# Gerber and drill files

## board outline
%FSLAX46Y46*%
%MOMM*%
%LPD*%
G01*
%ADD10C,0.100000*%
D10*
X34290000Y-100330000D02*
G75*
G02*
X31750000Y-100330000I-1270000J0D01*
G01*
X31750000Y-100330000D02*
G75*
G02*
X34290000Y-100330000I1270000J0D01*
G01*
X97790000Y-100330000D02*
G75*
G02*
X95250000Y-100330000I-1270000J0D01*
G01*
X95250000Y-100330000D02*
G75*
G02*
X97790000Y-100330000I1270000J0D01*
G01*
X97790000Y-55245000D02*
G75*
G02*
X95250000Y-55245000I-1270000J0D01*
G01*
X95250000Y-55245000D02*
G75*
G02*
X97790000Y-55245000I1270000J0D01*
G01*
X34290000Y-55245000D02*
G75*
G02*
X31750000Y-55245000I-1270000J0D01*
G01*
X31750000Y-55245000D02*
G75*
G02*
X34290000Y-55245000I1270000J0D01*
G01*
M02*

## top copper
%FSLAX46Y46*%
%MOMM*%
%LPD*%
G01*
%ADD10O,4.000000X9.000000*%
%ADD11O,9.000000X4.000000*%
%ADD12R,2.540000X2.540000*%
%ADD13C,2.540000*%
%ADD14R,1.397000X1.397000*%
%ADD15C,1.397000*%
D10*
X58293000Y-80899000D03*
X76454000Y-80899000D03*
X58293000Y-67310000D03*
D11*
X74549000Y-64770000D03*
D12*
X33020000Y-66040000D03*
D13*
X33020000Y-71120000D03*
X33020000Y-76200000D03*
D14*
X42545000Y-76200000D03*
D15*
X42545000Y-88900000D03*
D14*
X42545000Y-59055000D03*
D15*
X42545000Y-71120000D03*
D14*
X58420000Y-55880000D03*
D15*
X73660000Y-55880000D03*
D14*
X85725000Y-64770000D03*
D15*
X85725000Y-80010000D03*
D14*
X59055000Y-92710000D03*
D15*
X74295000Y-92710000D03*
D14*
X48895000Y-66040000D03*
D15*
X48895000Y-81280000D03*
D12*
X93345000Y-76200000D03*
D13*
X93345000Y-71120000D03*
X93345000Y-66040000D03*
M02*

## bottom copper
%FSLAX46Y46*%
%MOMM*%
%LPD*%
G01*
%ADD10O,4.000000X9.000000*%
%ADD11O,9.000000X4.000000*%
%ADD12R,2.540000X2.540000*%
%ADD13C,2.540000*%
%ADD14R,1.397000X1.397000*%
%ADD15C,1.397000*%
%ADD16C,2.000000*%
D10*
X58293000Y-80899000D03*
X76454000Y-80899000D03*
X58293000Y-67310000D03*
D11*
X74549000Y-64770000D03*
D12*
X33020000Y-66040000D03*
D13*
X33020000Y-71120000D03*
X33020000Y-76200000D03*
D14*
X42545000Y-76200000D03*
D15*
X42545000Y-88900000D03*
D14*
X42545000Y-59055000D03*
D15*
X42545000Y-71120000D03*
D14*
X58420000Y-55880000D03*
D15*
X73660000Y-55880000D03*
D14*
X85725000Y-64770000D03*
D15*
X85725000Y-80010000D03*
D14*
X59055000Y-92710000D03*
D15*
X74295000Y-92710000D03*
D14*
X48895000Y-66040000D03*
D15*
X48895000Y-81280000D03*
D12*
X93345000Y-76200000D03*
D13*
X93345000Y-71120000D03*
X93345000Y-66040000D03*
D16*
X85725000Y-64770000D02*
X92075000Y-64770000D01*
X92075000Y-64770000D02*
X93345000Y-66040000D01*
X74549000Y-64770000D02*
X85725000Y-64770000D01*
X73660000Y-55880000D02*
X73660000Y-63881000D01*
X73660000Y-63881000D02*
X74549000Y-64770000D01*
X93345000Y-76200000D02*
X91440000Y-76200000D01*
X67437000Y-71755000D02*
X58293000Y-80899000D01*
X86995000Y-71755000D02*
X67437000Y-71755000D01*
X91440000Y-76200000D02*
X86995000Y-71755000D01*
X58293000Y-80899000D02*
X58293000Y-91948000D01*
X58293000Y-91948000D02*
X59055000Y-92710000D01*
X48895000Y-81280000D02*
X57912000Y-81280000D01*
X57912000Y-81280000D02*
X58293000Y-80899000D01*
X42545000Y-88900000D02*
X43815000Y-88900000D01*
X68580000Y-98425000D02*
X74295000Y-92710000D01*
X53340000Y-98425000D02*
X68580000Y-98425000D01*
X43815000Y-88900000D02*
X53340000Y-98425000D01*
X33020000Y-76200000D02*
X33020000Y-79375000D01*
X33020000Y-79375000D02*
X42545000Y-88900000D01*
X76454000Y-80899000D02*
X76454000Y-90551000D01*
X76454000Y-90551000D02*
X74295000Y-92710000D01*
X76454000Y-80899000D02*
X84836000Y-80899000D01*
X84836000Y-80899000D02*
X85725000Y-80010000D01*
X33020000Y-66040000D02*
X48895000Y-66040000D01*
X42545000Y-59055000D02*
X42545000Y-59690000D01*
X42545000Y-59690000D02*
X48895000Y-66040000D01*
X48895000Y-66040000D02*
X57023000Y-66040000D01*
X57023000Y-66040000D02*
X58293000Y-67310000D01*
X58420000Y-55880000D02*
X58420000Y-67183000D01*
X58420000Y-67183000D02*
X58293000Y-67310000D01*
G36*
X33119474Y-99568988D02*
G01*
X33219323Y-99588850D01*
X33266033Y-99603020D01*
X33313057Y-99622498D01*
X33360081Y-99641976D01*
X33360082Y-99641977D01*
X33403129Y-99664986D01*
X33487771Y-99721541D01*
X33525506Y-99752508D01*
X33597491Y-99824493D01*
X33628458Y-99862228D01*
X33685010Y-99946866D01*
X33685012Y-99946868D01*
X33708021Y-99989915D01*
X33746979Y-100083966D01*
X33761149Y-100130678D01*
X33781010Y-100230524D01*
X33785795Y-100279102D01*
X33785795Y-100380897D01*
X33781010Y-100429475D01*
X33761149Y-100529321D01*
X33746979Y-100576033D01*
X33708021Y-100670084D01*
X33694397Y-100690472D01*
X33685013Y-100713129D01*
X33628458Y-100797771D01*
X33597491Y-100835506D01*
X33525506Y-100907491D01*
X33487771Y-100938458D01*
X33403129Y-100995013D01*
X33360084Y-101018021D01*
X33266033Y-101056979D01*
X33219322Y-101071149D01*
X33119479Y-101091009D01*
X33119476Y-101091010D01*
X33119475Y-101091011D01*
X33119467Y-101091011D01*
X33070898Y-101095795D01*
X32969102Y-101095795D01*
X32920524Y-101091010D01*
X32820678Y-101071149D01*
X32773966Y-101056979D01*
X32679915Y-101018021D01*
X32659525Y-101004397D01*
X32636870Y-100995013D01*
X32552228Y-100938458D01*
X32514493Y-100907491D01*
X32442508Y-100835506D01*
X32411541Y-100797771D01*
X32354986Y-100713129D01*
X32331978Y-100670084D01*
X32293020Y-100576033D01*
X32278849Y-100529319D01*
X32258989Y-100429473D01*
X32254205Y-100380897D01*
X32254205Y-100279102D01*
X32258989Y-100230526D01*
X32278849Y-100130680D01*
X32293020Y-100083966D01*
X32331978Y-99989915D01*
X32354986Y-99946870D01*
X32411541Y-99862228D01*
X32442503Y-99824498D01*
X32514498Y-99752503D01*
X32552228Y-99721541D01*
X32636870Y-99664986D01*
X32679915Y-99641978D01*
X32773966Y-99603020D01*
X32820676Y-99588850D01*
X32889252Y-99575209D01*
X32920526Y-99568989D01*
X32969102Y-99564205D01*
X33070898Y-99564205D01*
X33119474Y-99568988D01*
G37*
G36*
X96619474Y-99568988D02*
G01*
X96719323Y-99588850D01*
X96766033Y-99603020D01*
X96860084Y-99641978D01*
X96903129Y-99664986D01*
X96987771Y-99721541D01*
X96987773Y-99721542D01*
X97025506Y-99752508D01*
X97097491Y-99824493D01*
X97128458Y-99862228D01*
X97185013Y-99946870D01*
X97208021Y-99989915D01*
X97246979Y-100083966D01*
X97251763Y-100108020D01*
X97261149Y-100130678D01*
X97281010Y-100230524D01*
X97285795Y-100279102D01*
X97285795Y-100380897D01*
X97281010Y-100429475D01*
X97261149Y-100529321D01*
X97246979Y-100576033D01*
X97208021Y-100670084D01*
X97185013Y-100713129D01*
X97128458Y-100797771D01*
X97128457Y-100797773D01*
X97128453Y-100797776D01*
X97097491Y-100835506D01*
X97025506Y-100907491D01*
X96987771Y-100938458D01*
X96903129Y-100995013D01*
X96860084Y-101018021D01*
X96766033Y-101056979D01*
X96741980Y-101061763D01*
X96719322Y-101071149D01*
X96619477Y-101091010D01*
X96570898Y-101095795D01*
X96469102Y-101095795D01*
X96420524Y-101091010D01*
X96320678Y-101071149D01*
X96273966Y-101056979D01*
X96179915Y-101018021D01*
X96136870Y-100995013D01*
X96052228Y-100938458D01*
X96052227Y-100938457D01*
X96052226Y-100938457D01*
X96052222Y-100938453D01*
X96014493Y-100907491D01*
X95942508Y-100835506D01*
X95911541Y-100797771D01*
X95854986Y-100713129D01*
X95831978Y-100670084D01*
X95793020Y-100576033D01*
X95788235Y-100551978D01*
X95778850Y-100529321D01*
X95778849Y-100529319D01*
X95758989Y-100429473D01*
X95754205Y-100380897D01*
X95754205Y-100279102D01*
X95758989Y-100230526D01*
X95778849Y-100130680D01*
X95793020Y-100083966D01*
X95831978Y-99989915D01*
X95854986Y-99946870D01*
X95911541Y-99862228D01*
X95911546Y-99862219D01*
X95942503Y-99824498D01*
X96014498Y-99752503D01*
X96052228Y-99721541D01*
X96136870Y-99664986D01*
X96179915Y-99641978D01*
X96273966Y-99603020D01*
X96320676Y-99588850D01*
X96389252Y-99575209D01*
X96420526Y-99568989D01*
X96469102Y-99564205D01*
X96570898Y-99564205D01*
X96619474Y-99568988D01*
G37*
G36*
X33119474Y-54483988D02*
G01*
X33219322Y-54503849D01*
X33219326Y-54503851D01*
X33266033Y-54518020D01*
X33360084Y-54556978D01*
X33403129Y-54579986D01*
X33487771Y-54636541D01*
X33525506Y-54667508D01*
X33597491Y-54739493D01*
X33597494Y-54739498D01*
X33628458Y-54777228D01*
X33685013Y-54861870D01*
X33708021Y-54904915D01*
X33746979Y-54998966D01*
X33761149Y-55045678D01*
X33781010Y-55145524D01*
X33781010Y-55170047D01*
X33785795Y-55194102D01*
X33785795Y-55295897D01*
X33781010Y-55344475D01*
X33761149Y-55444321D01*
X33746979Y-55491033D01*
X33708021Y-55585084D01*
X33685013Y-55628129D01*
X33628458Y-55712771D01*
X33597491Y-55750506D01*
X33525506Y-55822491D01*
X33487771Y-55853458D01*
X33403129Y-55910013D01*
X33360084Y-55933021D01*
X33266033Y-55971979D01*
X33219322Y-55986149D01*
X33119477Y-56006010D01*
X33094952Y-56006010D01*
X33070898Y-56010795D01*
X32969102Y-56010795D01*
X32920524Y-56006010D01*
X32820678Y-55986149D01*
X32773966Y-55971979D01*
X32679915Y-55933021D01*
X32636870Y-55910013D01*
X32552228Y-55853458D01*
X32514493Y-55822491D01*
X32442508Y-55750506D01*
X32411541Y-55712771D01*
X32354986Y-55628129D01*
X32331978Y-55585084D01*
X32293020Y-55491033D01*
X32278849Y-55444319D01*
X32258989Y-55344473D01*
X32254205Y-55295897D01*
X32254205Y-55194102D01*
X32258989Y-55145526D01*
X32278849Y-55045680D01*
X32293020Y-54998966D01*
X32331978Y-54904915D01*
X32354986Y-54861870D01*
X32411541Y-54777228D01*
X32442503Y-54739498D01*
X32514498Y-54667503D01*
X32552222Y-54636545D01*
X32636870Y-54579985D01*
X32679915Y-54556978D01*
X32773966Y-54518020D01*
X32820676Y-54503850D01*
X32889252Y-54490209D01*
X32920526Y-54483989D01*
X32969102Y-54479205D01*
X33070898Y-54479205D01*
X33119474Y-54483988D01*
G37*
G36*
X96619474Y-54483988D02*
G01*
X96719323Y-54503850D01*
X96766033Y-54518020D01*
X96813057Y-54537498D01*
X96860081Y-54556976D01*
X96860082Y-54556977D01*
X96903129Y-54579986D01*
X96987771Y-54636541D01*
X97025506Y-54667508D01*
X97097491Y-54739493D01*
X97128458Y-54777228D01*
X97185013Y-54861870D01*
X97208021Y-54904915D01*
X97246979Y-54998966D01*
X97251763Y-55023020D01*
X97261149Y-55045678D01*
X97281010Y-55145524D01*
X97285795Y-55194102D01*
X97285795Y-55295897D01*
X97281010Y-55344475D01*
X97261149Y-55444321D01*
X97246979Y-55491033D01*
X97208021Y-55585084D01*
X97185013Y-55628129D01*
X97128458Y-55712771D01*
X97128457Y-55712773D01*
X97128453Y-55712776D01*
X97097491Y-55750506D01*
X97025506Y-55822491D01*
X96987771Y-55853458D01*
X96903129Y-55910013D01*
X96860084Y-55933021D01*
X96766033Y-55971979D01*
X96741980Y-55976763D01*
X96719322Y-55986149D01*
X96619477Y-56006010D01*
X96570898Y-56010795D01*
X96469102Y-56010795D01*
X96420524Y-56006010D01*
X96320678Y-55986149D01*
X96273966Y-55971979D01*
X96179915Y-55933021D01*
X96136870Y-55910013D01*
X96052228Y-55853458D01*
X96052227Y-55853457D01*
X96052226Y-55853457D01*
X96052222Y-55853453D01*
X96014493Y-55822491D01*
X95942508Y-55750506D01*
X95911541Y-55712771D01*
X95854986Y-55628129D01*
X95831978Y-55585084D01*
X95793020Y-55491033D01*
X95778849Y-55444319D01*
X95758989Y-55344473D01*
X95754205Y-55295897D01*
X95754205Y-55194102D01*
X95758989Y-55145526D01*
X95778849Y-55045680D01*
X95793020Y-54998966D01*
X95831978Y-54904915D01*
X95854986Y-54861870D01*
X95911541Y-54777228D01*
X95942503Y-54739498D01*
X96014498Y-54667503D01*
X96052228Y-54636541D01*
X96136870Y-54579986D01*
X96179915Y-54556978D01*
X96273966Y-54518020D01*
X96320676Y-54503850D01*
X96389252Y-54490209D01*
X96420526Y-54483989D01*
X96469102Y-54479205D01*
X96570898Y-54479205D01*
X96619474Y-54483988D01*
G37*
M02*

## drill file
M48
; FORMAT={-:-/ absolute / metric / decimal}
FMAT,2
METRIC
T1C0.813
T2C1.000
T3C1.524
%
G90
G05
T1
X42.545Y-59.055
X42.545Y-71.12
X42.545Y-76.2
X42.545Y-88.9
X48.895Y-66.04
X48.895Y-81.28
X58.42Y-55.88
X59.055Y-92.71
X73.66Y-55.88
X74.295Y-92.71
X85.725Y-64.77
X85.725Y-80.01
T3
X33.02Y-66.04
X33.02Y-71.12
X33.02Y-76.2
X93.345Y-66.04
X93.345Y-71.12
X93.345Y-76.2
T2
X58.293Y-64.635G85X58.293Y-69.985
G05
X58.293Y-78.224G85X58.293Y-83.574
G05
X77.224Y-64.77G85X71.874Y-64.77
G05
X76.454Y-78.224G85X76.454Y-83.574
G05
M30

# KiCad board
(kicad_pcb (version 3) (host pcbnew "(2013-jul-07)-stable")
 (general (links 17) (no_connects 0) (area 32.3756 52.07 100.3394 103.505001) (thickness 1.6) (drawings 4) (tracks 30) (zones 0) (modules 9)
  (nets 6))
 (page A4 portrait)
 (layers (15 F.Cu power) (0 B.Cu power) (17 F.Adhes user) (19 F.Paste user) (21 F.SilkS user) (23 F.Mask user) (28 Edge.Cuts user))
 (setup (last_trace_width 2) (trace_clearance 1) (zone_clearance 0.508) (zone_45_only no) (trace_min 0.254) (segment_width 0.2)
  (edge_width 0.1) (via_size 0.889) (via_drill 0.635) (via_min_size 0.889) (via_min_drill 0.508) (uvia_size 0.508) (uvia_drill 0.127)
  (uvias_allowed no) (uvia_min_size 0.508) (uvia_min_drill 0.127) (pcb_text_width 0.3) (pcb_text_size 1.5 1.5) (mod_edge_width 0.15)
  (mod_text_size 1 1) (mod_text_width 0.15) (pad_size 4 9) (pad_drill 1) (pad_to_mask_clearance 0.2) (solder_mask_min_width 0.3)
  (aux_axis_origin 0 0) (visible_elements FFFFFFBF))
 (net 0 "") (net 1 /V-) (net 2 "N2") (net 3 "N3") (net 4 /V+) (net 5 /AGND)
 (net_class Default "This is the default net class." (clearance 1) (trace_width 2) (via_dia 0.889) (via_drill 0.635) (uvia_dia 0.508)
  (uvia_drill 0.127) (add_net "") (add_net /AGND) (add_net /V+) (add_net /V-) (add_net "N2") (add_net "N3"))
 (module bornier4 (layer F.Cu) (at 65.405 73.279 90)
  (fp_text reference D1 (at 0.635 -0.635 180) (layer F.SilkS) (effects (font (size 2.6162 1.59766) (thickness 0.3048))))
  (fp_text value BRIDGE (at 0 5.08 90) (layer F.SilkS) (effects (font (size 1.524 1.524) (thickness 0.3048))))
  (pad 1 thru_hole oval (at -7.62 -7.112 270) (size 9 4) (drill oval 6.35 1) (layers *.Cu *.Mask F.SilkS) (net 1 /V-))
  (pad 2 thru_hole oval (at -7.62 11.049 270) (size 9 4) (drill oval 6.35 1) (layers *.Cu *.Mask F.SilkS) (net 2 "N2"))
  (pad 4 thru_hole oval (at 5.969 -7.112 270) (size 9 4) (drill oval 6.35 1) (layers *.Cu *.Mask F.SilkS) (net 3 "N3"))
  (pad 3 thru_hole oval (at 8.509 9.144 270) (size 4 9) (drill oval 1 6.35) (layers *.Cu *.Mask F.SilkS) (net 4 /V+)))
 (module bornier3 (layer F.Cu) (at 33.02 71.12 270)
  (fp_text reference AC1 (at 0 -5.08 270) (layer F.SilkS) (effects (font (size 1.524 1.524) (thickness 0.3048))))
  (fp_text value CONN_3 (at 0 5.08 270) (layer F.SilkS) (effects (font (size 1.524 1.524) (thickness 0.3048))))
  (pad 1 thru_hole rect (at -5.08 0 270) (size 2.54 2.54) (drill 1.524) (layers *.Cu *.Mask F.SilkS) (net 3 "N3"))
  (pad 2 thru_hole circle (at 0 0 270) (size 2.54 2.54) (drill 1.524) (layers *.Cu *.Mask F.SilkS) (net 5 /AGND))
  (pad 3 thru_hole circle (at 5.08 0 270) (size 2.54 2.54) (drill 1.524) (layers *.Cu *.Mask F.SilkS) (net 2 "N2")))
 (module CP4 (layer F.Cu) (at 42.545 81.28 270)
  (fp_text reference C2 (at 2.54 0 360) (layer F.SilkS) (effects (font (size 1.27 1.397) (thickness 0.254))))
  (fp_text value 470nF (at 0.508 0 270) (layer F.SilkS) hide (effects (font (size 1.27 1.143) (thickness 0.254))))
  (pad 1 thru_hole rect (at -5.08 0 270) (size 1.397 1.397) (drill 0.8128) (layers *.Cu *.Mask F.SilkS) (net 5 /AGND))
  (pad 2 thru_hole circle (at 7.62 0 270) (size 1.397 1.397) (drill 0.8128) (layers *.Cu *.Mask F.SilkS) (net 2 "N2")))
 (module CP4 (layer F.Cu) (at 42.545 66.04 270)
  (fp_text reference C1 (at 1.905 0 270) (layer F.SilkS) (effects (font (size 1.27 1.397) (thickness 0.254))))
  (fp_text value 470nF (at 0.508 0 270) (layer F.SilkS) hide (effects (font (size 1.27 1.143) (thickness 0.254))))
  (pad 1 thru_hole rect (at -6.985 0 270) (size 1.397 1.397) (drill 0.8128) (layers *.Cu *.Mask F.SilkS) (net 3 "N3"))
  (pad 2 thru_hole circle (at 5.08 0 270) (size 1.397 1.397) (drill 0.8128) (layers *.Cu *.Mask F.SilkS) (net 5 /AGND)))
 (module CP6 (layer F.Cu) (at 66.04 55.88)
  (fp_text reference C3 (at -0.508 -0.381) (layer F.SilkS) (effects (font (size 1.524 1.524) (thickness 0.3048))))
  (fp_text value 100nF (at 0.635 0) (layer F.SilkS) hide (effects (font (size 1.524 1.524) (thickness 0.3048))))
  (pad 1 thru_hole rect (at -7.62 0) (size 1.397 1.397) (drill 0.8128) (layers *.Cu *.Mask F.SilkS) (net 3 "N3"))
  (pad 2 thru_hole circle (at 7.62 0) (size 1.397 1.397) (drill 0.8128) (layers *.Cu *.Mask F.SilkS) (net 4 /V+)))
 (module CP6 (layer F.Cu) (at 85.725 72.39 270)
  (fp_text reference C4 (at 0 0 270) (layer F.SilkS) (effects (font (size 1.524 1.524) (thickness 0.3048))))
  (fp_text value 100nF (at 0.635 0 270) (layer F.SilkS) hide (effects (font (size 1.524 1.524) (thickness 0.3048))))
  (pad 1 thru_hole rect (at -7.62 0 270) (size 1.397 1.397) (drill 0.8128) (layers *.Cu *.Mask F.SilkS) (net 4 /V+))
  (pad 2 thru_hole circle (at 7.62 0 270) (size 1.397 1.397) (drill 0.8128) (layers *.Cu *.Mask F.SilkS) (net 2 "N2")))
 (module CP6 (layer F.Cu) (at 66.675 92.71)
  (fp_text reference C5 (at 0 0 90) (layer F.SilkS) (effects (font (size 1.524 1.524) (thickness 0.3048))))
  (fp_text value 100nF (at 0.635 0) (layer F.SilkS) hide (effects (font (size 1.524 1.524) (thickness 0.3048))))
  (pad 1 thru_hole rect (at -7.62 0) (size 1.397 1.397) (drill 0.8128) (layers *.Cu *.Mask F.SilkS) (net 1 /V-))
  (pad 2 thru_hole circle (at 7.62 0) (size 1.397 1.397) (drill 0.8128) (layers *.Cu *.Mask F.SilkS) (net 2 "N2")))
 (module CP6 (layer F.Cu) (at 48.895 73.66 270)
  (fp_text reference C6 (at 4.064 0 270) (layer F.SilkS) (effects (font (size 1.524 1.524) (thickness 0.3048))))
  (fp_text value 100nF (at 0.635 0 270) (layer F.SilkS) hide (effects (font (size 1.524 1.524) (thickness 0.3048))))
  (pad 1 thru_hole rect (at -7.62 0 270) (size 1.397 1.397) (drill 0.8128) (layers *.Cu *.Mask F.SilkS) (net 3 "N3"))
  (pad 2 thru_hole circle (at 7.62 0 270) (size 1.397 1.397) (drill 0.8128) (layers *.Cu *.Mask F.SilkS) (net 1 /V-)))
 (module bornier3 (layer F.Cu) (at 93.345 71.12 90)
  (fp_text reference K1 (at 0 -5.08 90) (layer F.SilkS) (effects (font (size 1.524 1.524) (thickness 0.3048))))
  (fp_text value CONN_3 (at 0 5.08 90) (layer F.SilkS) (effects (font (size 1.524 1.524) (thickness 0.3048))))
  (pad 1 thru_hole rect (at -5.08 0 90) (size 2.54 2.54) (drill 1.524) (layers *.Cu *.Mask F.SilkS) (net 1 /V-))
  (pad 2 thru_hole circle (at 0 0 90) (size 2.54 2.54) (drill 1.524) (layers *.Cu *.Mask F.SilkS) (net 5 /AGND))
  (pad 3 thru_hole circle (at 5.08 0 90) (size 2.54 2.54) (drill 1.524) (layers *.Cu *.Mask F.SilkS) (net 4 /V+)))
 (gr_circle (center 33.02 100.33) (end 34.29 100.33) (layer Edge.Cuts) (width 0.1))
 (gr_circle (center 96.52 100.33) (end 97.79 100.33) (layer Edge.Cuts) (width 0.1))
 (gr_circle (center 96.52 55.245) (end 97.79 55.245) (layer Edge.Cuts) (width 0.1))
 (gr_circle (center 33.02 55.245) (end 34.29 55.245) (layer Edge.Cuts) (width 0.1))
 (segment (start 85.725 64.77) (end 92.075 64.77) (width 2) (layer B.Cu) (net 4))
 (segment (start 92.075 64.77) (end 93.345 66.04) (width 2) (layer B.Cu) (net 4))
 (segment (start 74.549 64.77) (end 85.725 64.77) (width 2) (layer B.Cu) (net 4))
 (segment (start 73.66 55.88) (end 73.66 63.881) (width 2) (layer B.Cu) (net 4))
 (segment (start 73.66 63.881) (end 74.549 64.77) (width 2) (layer B.Cu) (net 4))
 (segment (start 93.345 76.2) (end 91.44 76.2) (width 2) (layer B.Cu) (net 1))
 (segment (start 67.437 71.755) (end 58.293 80.899) (width 2) (layer B.Cu) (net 1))
 (segment (start 86.995 71.755) (end 67.437 71.755) (width 2) (layer B.Cu) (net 1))
 (segment (start 91.44 76.2) (end 86.995 71.755) (width 2) (layer B.Cu) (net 1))
 (segment (start 58.293 80.899) (end 58.293 91.948) (width 2) (layer B.Cu) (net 1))
 (segment (start 58.293 91.948) (end 59.055 92.71) (width 2) (layer B.Cu) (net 1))
 (segment (start 48.895 81.28) (end 57.912 81.28) (width 2) (layer B.Cu) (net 1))
 (segment (start 57.912 81.28) (end 58.293 80.899) (width 2) (layer B.Cu) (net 1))
 (segment (start 42.545 88.9) (end 43.815 88.9) (width 2) (layer B.Cu) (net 2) (status 400000))
 (segment (start 68.58 98.425) (end 74.295 92.71) (width 2) (layer B.Cu) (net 2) (status 800000))
 (segment (start 53.34 98.425) (end 68.58 98.425) (width 2) (layer B.Cu) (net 2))
 (segment (start 43.815 88.9) (end 53.34 98.425) (width 2) (layer B.Cu) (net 2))
 (segment (start 33.02 76.2) (end 33.02 79.375) (width 2) (layer B.Cu) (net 2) (status 400000))
 (segment (start 33.02 79.375) (end 42.545 88.9) (width 2) (layer B.Cu) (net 2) (status 800000))
 (segment (start 76.454 80.899) (end 76.454 90.551) (width 2) (layer B.Cu) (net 2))
 (segment (start 76.454 90.551) (end 74.295 92.71) (width 2) (layer B.Cu) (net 2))
 (segment (start 76.454 80.899) (end 84.836 80.899) (width 2) (layer B.Cu) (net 2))
 (segment (start 84.836 80.899) (end 85.725 80.01) (width 2) (layer B.Cu) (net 2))
 (segment (start 33.02 66.04) (end 48.895 66.04) (width 2) (layer B.Cu) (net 3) (status C00000))
 (segment (start 42.545 59.055) (end 42.545 59.69) (width 2) (layer B.Cu) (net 3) (status C00000))
 (segment (start 42.545 59.69) (end 48.895 66.04) (width 2) (layer B.Cu) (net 3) (status C00000))
 (segment (start 48.895 66.04) (end 57.023 66.04) (width 2) (layer B.Cu) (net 3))
 (segment (start 57.023 66.04) (end 58.293 67.31) (width 2) (layer B.Cu) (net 3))
 (segment (start 58.42 55.88) (end 58.42 67.183) (width 2) (layer B.Cu) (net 3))
 (segment (start 58.42 67.183) (end 58.293 67.31) (width 2) (layer B.Cu) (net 3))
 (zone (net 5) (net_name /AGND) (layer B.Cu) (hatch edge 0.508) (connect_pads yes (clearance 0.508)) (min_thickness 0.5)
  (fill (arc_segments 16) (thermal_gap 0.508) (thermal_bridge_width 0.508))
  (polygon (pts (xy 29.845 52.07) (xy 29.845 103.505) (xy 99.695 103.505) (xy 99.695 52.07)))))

